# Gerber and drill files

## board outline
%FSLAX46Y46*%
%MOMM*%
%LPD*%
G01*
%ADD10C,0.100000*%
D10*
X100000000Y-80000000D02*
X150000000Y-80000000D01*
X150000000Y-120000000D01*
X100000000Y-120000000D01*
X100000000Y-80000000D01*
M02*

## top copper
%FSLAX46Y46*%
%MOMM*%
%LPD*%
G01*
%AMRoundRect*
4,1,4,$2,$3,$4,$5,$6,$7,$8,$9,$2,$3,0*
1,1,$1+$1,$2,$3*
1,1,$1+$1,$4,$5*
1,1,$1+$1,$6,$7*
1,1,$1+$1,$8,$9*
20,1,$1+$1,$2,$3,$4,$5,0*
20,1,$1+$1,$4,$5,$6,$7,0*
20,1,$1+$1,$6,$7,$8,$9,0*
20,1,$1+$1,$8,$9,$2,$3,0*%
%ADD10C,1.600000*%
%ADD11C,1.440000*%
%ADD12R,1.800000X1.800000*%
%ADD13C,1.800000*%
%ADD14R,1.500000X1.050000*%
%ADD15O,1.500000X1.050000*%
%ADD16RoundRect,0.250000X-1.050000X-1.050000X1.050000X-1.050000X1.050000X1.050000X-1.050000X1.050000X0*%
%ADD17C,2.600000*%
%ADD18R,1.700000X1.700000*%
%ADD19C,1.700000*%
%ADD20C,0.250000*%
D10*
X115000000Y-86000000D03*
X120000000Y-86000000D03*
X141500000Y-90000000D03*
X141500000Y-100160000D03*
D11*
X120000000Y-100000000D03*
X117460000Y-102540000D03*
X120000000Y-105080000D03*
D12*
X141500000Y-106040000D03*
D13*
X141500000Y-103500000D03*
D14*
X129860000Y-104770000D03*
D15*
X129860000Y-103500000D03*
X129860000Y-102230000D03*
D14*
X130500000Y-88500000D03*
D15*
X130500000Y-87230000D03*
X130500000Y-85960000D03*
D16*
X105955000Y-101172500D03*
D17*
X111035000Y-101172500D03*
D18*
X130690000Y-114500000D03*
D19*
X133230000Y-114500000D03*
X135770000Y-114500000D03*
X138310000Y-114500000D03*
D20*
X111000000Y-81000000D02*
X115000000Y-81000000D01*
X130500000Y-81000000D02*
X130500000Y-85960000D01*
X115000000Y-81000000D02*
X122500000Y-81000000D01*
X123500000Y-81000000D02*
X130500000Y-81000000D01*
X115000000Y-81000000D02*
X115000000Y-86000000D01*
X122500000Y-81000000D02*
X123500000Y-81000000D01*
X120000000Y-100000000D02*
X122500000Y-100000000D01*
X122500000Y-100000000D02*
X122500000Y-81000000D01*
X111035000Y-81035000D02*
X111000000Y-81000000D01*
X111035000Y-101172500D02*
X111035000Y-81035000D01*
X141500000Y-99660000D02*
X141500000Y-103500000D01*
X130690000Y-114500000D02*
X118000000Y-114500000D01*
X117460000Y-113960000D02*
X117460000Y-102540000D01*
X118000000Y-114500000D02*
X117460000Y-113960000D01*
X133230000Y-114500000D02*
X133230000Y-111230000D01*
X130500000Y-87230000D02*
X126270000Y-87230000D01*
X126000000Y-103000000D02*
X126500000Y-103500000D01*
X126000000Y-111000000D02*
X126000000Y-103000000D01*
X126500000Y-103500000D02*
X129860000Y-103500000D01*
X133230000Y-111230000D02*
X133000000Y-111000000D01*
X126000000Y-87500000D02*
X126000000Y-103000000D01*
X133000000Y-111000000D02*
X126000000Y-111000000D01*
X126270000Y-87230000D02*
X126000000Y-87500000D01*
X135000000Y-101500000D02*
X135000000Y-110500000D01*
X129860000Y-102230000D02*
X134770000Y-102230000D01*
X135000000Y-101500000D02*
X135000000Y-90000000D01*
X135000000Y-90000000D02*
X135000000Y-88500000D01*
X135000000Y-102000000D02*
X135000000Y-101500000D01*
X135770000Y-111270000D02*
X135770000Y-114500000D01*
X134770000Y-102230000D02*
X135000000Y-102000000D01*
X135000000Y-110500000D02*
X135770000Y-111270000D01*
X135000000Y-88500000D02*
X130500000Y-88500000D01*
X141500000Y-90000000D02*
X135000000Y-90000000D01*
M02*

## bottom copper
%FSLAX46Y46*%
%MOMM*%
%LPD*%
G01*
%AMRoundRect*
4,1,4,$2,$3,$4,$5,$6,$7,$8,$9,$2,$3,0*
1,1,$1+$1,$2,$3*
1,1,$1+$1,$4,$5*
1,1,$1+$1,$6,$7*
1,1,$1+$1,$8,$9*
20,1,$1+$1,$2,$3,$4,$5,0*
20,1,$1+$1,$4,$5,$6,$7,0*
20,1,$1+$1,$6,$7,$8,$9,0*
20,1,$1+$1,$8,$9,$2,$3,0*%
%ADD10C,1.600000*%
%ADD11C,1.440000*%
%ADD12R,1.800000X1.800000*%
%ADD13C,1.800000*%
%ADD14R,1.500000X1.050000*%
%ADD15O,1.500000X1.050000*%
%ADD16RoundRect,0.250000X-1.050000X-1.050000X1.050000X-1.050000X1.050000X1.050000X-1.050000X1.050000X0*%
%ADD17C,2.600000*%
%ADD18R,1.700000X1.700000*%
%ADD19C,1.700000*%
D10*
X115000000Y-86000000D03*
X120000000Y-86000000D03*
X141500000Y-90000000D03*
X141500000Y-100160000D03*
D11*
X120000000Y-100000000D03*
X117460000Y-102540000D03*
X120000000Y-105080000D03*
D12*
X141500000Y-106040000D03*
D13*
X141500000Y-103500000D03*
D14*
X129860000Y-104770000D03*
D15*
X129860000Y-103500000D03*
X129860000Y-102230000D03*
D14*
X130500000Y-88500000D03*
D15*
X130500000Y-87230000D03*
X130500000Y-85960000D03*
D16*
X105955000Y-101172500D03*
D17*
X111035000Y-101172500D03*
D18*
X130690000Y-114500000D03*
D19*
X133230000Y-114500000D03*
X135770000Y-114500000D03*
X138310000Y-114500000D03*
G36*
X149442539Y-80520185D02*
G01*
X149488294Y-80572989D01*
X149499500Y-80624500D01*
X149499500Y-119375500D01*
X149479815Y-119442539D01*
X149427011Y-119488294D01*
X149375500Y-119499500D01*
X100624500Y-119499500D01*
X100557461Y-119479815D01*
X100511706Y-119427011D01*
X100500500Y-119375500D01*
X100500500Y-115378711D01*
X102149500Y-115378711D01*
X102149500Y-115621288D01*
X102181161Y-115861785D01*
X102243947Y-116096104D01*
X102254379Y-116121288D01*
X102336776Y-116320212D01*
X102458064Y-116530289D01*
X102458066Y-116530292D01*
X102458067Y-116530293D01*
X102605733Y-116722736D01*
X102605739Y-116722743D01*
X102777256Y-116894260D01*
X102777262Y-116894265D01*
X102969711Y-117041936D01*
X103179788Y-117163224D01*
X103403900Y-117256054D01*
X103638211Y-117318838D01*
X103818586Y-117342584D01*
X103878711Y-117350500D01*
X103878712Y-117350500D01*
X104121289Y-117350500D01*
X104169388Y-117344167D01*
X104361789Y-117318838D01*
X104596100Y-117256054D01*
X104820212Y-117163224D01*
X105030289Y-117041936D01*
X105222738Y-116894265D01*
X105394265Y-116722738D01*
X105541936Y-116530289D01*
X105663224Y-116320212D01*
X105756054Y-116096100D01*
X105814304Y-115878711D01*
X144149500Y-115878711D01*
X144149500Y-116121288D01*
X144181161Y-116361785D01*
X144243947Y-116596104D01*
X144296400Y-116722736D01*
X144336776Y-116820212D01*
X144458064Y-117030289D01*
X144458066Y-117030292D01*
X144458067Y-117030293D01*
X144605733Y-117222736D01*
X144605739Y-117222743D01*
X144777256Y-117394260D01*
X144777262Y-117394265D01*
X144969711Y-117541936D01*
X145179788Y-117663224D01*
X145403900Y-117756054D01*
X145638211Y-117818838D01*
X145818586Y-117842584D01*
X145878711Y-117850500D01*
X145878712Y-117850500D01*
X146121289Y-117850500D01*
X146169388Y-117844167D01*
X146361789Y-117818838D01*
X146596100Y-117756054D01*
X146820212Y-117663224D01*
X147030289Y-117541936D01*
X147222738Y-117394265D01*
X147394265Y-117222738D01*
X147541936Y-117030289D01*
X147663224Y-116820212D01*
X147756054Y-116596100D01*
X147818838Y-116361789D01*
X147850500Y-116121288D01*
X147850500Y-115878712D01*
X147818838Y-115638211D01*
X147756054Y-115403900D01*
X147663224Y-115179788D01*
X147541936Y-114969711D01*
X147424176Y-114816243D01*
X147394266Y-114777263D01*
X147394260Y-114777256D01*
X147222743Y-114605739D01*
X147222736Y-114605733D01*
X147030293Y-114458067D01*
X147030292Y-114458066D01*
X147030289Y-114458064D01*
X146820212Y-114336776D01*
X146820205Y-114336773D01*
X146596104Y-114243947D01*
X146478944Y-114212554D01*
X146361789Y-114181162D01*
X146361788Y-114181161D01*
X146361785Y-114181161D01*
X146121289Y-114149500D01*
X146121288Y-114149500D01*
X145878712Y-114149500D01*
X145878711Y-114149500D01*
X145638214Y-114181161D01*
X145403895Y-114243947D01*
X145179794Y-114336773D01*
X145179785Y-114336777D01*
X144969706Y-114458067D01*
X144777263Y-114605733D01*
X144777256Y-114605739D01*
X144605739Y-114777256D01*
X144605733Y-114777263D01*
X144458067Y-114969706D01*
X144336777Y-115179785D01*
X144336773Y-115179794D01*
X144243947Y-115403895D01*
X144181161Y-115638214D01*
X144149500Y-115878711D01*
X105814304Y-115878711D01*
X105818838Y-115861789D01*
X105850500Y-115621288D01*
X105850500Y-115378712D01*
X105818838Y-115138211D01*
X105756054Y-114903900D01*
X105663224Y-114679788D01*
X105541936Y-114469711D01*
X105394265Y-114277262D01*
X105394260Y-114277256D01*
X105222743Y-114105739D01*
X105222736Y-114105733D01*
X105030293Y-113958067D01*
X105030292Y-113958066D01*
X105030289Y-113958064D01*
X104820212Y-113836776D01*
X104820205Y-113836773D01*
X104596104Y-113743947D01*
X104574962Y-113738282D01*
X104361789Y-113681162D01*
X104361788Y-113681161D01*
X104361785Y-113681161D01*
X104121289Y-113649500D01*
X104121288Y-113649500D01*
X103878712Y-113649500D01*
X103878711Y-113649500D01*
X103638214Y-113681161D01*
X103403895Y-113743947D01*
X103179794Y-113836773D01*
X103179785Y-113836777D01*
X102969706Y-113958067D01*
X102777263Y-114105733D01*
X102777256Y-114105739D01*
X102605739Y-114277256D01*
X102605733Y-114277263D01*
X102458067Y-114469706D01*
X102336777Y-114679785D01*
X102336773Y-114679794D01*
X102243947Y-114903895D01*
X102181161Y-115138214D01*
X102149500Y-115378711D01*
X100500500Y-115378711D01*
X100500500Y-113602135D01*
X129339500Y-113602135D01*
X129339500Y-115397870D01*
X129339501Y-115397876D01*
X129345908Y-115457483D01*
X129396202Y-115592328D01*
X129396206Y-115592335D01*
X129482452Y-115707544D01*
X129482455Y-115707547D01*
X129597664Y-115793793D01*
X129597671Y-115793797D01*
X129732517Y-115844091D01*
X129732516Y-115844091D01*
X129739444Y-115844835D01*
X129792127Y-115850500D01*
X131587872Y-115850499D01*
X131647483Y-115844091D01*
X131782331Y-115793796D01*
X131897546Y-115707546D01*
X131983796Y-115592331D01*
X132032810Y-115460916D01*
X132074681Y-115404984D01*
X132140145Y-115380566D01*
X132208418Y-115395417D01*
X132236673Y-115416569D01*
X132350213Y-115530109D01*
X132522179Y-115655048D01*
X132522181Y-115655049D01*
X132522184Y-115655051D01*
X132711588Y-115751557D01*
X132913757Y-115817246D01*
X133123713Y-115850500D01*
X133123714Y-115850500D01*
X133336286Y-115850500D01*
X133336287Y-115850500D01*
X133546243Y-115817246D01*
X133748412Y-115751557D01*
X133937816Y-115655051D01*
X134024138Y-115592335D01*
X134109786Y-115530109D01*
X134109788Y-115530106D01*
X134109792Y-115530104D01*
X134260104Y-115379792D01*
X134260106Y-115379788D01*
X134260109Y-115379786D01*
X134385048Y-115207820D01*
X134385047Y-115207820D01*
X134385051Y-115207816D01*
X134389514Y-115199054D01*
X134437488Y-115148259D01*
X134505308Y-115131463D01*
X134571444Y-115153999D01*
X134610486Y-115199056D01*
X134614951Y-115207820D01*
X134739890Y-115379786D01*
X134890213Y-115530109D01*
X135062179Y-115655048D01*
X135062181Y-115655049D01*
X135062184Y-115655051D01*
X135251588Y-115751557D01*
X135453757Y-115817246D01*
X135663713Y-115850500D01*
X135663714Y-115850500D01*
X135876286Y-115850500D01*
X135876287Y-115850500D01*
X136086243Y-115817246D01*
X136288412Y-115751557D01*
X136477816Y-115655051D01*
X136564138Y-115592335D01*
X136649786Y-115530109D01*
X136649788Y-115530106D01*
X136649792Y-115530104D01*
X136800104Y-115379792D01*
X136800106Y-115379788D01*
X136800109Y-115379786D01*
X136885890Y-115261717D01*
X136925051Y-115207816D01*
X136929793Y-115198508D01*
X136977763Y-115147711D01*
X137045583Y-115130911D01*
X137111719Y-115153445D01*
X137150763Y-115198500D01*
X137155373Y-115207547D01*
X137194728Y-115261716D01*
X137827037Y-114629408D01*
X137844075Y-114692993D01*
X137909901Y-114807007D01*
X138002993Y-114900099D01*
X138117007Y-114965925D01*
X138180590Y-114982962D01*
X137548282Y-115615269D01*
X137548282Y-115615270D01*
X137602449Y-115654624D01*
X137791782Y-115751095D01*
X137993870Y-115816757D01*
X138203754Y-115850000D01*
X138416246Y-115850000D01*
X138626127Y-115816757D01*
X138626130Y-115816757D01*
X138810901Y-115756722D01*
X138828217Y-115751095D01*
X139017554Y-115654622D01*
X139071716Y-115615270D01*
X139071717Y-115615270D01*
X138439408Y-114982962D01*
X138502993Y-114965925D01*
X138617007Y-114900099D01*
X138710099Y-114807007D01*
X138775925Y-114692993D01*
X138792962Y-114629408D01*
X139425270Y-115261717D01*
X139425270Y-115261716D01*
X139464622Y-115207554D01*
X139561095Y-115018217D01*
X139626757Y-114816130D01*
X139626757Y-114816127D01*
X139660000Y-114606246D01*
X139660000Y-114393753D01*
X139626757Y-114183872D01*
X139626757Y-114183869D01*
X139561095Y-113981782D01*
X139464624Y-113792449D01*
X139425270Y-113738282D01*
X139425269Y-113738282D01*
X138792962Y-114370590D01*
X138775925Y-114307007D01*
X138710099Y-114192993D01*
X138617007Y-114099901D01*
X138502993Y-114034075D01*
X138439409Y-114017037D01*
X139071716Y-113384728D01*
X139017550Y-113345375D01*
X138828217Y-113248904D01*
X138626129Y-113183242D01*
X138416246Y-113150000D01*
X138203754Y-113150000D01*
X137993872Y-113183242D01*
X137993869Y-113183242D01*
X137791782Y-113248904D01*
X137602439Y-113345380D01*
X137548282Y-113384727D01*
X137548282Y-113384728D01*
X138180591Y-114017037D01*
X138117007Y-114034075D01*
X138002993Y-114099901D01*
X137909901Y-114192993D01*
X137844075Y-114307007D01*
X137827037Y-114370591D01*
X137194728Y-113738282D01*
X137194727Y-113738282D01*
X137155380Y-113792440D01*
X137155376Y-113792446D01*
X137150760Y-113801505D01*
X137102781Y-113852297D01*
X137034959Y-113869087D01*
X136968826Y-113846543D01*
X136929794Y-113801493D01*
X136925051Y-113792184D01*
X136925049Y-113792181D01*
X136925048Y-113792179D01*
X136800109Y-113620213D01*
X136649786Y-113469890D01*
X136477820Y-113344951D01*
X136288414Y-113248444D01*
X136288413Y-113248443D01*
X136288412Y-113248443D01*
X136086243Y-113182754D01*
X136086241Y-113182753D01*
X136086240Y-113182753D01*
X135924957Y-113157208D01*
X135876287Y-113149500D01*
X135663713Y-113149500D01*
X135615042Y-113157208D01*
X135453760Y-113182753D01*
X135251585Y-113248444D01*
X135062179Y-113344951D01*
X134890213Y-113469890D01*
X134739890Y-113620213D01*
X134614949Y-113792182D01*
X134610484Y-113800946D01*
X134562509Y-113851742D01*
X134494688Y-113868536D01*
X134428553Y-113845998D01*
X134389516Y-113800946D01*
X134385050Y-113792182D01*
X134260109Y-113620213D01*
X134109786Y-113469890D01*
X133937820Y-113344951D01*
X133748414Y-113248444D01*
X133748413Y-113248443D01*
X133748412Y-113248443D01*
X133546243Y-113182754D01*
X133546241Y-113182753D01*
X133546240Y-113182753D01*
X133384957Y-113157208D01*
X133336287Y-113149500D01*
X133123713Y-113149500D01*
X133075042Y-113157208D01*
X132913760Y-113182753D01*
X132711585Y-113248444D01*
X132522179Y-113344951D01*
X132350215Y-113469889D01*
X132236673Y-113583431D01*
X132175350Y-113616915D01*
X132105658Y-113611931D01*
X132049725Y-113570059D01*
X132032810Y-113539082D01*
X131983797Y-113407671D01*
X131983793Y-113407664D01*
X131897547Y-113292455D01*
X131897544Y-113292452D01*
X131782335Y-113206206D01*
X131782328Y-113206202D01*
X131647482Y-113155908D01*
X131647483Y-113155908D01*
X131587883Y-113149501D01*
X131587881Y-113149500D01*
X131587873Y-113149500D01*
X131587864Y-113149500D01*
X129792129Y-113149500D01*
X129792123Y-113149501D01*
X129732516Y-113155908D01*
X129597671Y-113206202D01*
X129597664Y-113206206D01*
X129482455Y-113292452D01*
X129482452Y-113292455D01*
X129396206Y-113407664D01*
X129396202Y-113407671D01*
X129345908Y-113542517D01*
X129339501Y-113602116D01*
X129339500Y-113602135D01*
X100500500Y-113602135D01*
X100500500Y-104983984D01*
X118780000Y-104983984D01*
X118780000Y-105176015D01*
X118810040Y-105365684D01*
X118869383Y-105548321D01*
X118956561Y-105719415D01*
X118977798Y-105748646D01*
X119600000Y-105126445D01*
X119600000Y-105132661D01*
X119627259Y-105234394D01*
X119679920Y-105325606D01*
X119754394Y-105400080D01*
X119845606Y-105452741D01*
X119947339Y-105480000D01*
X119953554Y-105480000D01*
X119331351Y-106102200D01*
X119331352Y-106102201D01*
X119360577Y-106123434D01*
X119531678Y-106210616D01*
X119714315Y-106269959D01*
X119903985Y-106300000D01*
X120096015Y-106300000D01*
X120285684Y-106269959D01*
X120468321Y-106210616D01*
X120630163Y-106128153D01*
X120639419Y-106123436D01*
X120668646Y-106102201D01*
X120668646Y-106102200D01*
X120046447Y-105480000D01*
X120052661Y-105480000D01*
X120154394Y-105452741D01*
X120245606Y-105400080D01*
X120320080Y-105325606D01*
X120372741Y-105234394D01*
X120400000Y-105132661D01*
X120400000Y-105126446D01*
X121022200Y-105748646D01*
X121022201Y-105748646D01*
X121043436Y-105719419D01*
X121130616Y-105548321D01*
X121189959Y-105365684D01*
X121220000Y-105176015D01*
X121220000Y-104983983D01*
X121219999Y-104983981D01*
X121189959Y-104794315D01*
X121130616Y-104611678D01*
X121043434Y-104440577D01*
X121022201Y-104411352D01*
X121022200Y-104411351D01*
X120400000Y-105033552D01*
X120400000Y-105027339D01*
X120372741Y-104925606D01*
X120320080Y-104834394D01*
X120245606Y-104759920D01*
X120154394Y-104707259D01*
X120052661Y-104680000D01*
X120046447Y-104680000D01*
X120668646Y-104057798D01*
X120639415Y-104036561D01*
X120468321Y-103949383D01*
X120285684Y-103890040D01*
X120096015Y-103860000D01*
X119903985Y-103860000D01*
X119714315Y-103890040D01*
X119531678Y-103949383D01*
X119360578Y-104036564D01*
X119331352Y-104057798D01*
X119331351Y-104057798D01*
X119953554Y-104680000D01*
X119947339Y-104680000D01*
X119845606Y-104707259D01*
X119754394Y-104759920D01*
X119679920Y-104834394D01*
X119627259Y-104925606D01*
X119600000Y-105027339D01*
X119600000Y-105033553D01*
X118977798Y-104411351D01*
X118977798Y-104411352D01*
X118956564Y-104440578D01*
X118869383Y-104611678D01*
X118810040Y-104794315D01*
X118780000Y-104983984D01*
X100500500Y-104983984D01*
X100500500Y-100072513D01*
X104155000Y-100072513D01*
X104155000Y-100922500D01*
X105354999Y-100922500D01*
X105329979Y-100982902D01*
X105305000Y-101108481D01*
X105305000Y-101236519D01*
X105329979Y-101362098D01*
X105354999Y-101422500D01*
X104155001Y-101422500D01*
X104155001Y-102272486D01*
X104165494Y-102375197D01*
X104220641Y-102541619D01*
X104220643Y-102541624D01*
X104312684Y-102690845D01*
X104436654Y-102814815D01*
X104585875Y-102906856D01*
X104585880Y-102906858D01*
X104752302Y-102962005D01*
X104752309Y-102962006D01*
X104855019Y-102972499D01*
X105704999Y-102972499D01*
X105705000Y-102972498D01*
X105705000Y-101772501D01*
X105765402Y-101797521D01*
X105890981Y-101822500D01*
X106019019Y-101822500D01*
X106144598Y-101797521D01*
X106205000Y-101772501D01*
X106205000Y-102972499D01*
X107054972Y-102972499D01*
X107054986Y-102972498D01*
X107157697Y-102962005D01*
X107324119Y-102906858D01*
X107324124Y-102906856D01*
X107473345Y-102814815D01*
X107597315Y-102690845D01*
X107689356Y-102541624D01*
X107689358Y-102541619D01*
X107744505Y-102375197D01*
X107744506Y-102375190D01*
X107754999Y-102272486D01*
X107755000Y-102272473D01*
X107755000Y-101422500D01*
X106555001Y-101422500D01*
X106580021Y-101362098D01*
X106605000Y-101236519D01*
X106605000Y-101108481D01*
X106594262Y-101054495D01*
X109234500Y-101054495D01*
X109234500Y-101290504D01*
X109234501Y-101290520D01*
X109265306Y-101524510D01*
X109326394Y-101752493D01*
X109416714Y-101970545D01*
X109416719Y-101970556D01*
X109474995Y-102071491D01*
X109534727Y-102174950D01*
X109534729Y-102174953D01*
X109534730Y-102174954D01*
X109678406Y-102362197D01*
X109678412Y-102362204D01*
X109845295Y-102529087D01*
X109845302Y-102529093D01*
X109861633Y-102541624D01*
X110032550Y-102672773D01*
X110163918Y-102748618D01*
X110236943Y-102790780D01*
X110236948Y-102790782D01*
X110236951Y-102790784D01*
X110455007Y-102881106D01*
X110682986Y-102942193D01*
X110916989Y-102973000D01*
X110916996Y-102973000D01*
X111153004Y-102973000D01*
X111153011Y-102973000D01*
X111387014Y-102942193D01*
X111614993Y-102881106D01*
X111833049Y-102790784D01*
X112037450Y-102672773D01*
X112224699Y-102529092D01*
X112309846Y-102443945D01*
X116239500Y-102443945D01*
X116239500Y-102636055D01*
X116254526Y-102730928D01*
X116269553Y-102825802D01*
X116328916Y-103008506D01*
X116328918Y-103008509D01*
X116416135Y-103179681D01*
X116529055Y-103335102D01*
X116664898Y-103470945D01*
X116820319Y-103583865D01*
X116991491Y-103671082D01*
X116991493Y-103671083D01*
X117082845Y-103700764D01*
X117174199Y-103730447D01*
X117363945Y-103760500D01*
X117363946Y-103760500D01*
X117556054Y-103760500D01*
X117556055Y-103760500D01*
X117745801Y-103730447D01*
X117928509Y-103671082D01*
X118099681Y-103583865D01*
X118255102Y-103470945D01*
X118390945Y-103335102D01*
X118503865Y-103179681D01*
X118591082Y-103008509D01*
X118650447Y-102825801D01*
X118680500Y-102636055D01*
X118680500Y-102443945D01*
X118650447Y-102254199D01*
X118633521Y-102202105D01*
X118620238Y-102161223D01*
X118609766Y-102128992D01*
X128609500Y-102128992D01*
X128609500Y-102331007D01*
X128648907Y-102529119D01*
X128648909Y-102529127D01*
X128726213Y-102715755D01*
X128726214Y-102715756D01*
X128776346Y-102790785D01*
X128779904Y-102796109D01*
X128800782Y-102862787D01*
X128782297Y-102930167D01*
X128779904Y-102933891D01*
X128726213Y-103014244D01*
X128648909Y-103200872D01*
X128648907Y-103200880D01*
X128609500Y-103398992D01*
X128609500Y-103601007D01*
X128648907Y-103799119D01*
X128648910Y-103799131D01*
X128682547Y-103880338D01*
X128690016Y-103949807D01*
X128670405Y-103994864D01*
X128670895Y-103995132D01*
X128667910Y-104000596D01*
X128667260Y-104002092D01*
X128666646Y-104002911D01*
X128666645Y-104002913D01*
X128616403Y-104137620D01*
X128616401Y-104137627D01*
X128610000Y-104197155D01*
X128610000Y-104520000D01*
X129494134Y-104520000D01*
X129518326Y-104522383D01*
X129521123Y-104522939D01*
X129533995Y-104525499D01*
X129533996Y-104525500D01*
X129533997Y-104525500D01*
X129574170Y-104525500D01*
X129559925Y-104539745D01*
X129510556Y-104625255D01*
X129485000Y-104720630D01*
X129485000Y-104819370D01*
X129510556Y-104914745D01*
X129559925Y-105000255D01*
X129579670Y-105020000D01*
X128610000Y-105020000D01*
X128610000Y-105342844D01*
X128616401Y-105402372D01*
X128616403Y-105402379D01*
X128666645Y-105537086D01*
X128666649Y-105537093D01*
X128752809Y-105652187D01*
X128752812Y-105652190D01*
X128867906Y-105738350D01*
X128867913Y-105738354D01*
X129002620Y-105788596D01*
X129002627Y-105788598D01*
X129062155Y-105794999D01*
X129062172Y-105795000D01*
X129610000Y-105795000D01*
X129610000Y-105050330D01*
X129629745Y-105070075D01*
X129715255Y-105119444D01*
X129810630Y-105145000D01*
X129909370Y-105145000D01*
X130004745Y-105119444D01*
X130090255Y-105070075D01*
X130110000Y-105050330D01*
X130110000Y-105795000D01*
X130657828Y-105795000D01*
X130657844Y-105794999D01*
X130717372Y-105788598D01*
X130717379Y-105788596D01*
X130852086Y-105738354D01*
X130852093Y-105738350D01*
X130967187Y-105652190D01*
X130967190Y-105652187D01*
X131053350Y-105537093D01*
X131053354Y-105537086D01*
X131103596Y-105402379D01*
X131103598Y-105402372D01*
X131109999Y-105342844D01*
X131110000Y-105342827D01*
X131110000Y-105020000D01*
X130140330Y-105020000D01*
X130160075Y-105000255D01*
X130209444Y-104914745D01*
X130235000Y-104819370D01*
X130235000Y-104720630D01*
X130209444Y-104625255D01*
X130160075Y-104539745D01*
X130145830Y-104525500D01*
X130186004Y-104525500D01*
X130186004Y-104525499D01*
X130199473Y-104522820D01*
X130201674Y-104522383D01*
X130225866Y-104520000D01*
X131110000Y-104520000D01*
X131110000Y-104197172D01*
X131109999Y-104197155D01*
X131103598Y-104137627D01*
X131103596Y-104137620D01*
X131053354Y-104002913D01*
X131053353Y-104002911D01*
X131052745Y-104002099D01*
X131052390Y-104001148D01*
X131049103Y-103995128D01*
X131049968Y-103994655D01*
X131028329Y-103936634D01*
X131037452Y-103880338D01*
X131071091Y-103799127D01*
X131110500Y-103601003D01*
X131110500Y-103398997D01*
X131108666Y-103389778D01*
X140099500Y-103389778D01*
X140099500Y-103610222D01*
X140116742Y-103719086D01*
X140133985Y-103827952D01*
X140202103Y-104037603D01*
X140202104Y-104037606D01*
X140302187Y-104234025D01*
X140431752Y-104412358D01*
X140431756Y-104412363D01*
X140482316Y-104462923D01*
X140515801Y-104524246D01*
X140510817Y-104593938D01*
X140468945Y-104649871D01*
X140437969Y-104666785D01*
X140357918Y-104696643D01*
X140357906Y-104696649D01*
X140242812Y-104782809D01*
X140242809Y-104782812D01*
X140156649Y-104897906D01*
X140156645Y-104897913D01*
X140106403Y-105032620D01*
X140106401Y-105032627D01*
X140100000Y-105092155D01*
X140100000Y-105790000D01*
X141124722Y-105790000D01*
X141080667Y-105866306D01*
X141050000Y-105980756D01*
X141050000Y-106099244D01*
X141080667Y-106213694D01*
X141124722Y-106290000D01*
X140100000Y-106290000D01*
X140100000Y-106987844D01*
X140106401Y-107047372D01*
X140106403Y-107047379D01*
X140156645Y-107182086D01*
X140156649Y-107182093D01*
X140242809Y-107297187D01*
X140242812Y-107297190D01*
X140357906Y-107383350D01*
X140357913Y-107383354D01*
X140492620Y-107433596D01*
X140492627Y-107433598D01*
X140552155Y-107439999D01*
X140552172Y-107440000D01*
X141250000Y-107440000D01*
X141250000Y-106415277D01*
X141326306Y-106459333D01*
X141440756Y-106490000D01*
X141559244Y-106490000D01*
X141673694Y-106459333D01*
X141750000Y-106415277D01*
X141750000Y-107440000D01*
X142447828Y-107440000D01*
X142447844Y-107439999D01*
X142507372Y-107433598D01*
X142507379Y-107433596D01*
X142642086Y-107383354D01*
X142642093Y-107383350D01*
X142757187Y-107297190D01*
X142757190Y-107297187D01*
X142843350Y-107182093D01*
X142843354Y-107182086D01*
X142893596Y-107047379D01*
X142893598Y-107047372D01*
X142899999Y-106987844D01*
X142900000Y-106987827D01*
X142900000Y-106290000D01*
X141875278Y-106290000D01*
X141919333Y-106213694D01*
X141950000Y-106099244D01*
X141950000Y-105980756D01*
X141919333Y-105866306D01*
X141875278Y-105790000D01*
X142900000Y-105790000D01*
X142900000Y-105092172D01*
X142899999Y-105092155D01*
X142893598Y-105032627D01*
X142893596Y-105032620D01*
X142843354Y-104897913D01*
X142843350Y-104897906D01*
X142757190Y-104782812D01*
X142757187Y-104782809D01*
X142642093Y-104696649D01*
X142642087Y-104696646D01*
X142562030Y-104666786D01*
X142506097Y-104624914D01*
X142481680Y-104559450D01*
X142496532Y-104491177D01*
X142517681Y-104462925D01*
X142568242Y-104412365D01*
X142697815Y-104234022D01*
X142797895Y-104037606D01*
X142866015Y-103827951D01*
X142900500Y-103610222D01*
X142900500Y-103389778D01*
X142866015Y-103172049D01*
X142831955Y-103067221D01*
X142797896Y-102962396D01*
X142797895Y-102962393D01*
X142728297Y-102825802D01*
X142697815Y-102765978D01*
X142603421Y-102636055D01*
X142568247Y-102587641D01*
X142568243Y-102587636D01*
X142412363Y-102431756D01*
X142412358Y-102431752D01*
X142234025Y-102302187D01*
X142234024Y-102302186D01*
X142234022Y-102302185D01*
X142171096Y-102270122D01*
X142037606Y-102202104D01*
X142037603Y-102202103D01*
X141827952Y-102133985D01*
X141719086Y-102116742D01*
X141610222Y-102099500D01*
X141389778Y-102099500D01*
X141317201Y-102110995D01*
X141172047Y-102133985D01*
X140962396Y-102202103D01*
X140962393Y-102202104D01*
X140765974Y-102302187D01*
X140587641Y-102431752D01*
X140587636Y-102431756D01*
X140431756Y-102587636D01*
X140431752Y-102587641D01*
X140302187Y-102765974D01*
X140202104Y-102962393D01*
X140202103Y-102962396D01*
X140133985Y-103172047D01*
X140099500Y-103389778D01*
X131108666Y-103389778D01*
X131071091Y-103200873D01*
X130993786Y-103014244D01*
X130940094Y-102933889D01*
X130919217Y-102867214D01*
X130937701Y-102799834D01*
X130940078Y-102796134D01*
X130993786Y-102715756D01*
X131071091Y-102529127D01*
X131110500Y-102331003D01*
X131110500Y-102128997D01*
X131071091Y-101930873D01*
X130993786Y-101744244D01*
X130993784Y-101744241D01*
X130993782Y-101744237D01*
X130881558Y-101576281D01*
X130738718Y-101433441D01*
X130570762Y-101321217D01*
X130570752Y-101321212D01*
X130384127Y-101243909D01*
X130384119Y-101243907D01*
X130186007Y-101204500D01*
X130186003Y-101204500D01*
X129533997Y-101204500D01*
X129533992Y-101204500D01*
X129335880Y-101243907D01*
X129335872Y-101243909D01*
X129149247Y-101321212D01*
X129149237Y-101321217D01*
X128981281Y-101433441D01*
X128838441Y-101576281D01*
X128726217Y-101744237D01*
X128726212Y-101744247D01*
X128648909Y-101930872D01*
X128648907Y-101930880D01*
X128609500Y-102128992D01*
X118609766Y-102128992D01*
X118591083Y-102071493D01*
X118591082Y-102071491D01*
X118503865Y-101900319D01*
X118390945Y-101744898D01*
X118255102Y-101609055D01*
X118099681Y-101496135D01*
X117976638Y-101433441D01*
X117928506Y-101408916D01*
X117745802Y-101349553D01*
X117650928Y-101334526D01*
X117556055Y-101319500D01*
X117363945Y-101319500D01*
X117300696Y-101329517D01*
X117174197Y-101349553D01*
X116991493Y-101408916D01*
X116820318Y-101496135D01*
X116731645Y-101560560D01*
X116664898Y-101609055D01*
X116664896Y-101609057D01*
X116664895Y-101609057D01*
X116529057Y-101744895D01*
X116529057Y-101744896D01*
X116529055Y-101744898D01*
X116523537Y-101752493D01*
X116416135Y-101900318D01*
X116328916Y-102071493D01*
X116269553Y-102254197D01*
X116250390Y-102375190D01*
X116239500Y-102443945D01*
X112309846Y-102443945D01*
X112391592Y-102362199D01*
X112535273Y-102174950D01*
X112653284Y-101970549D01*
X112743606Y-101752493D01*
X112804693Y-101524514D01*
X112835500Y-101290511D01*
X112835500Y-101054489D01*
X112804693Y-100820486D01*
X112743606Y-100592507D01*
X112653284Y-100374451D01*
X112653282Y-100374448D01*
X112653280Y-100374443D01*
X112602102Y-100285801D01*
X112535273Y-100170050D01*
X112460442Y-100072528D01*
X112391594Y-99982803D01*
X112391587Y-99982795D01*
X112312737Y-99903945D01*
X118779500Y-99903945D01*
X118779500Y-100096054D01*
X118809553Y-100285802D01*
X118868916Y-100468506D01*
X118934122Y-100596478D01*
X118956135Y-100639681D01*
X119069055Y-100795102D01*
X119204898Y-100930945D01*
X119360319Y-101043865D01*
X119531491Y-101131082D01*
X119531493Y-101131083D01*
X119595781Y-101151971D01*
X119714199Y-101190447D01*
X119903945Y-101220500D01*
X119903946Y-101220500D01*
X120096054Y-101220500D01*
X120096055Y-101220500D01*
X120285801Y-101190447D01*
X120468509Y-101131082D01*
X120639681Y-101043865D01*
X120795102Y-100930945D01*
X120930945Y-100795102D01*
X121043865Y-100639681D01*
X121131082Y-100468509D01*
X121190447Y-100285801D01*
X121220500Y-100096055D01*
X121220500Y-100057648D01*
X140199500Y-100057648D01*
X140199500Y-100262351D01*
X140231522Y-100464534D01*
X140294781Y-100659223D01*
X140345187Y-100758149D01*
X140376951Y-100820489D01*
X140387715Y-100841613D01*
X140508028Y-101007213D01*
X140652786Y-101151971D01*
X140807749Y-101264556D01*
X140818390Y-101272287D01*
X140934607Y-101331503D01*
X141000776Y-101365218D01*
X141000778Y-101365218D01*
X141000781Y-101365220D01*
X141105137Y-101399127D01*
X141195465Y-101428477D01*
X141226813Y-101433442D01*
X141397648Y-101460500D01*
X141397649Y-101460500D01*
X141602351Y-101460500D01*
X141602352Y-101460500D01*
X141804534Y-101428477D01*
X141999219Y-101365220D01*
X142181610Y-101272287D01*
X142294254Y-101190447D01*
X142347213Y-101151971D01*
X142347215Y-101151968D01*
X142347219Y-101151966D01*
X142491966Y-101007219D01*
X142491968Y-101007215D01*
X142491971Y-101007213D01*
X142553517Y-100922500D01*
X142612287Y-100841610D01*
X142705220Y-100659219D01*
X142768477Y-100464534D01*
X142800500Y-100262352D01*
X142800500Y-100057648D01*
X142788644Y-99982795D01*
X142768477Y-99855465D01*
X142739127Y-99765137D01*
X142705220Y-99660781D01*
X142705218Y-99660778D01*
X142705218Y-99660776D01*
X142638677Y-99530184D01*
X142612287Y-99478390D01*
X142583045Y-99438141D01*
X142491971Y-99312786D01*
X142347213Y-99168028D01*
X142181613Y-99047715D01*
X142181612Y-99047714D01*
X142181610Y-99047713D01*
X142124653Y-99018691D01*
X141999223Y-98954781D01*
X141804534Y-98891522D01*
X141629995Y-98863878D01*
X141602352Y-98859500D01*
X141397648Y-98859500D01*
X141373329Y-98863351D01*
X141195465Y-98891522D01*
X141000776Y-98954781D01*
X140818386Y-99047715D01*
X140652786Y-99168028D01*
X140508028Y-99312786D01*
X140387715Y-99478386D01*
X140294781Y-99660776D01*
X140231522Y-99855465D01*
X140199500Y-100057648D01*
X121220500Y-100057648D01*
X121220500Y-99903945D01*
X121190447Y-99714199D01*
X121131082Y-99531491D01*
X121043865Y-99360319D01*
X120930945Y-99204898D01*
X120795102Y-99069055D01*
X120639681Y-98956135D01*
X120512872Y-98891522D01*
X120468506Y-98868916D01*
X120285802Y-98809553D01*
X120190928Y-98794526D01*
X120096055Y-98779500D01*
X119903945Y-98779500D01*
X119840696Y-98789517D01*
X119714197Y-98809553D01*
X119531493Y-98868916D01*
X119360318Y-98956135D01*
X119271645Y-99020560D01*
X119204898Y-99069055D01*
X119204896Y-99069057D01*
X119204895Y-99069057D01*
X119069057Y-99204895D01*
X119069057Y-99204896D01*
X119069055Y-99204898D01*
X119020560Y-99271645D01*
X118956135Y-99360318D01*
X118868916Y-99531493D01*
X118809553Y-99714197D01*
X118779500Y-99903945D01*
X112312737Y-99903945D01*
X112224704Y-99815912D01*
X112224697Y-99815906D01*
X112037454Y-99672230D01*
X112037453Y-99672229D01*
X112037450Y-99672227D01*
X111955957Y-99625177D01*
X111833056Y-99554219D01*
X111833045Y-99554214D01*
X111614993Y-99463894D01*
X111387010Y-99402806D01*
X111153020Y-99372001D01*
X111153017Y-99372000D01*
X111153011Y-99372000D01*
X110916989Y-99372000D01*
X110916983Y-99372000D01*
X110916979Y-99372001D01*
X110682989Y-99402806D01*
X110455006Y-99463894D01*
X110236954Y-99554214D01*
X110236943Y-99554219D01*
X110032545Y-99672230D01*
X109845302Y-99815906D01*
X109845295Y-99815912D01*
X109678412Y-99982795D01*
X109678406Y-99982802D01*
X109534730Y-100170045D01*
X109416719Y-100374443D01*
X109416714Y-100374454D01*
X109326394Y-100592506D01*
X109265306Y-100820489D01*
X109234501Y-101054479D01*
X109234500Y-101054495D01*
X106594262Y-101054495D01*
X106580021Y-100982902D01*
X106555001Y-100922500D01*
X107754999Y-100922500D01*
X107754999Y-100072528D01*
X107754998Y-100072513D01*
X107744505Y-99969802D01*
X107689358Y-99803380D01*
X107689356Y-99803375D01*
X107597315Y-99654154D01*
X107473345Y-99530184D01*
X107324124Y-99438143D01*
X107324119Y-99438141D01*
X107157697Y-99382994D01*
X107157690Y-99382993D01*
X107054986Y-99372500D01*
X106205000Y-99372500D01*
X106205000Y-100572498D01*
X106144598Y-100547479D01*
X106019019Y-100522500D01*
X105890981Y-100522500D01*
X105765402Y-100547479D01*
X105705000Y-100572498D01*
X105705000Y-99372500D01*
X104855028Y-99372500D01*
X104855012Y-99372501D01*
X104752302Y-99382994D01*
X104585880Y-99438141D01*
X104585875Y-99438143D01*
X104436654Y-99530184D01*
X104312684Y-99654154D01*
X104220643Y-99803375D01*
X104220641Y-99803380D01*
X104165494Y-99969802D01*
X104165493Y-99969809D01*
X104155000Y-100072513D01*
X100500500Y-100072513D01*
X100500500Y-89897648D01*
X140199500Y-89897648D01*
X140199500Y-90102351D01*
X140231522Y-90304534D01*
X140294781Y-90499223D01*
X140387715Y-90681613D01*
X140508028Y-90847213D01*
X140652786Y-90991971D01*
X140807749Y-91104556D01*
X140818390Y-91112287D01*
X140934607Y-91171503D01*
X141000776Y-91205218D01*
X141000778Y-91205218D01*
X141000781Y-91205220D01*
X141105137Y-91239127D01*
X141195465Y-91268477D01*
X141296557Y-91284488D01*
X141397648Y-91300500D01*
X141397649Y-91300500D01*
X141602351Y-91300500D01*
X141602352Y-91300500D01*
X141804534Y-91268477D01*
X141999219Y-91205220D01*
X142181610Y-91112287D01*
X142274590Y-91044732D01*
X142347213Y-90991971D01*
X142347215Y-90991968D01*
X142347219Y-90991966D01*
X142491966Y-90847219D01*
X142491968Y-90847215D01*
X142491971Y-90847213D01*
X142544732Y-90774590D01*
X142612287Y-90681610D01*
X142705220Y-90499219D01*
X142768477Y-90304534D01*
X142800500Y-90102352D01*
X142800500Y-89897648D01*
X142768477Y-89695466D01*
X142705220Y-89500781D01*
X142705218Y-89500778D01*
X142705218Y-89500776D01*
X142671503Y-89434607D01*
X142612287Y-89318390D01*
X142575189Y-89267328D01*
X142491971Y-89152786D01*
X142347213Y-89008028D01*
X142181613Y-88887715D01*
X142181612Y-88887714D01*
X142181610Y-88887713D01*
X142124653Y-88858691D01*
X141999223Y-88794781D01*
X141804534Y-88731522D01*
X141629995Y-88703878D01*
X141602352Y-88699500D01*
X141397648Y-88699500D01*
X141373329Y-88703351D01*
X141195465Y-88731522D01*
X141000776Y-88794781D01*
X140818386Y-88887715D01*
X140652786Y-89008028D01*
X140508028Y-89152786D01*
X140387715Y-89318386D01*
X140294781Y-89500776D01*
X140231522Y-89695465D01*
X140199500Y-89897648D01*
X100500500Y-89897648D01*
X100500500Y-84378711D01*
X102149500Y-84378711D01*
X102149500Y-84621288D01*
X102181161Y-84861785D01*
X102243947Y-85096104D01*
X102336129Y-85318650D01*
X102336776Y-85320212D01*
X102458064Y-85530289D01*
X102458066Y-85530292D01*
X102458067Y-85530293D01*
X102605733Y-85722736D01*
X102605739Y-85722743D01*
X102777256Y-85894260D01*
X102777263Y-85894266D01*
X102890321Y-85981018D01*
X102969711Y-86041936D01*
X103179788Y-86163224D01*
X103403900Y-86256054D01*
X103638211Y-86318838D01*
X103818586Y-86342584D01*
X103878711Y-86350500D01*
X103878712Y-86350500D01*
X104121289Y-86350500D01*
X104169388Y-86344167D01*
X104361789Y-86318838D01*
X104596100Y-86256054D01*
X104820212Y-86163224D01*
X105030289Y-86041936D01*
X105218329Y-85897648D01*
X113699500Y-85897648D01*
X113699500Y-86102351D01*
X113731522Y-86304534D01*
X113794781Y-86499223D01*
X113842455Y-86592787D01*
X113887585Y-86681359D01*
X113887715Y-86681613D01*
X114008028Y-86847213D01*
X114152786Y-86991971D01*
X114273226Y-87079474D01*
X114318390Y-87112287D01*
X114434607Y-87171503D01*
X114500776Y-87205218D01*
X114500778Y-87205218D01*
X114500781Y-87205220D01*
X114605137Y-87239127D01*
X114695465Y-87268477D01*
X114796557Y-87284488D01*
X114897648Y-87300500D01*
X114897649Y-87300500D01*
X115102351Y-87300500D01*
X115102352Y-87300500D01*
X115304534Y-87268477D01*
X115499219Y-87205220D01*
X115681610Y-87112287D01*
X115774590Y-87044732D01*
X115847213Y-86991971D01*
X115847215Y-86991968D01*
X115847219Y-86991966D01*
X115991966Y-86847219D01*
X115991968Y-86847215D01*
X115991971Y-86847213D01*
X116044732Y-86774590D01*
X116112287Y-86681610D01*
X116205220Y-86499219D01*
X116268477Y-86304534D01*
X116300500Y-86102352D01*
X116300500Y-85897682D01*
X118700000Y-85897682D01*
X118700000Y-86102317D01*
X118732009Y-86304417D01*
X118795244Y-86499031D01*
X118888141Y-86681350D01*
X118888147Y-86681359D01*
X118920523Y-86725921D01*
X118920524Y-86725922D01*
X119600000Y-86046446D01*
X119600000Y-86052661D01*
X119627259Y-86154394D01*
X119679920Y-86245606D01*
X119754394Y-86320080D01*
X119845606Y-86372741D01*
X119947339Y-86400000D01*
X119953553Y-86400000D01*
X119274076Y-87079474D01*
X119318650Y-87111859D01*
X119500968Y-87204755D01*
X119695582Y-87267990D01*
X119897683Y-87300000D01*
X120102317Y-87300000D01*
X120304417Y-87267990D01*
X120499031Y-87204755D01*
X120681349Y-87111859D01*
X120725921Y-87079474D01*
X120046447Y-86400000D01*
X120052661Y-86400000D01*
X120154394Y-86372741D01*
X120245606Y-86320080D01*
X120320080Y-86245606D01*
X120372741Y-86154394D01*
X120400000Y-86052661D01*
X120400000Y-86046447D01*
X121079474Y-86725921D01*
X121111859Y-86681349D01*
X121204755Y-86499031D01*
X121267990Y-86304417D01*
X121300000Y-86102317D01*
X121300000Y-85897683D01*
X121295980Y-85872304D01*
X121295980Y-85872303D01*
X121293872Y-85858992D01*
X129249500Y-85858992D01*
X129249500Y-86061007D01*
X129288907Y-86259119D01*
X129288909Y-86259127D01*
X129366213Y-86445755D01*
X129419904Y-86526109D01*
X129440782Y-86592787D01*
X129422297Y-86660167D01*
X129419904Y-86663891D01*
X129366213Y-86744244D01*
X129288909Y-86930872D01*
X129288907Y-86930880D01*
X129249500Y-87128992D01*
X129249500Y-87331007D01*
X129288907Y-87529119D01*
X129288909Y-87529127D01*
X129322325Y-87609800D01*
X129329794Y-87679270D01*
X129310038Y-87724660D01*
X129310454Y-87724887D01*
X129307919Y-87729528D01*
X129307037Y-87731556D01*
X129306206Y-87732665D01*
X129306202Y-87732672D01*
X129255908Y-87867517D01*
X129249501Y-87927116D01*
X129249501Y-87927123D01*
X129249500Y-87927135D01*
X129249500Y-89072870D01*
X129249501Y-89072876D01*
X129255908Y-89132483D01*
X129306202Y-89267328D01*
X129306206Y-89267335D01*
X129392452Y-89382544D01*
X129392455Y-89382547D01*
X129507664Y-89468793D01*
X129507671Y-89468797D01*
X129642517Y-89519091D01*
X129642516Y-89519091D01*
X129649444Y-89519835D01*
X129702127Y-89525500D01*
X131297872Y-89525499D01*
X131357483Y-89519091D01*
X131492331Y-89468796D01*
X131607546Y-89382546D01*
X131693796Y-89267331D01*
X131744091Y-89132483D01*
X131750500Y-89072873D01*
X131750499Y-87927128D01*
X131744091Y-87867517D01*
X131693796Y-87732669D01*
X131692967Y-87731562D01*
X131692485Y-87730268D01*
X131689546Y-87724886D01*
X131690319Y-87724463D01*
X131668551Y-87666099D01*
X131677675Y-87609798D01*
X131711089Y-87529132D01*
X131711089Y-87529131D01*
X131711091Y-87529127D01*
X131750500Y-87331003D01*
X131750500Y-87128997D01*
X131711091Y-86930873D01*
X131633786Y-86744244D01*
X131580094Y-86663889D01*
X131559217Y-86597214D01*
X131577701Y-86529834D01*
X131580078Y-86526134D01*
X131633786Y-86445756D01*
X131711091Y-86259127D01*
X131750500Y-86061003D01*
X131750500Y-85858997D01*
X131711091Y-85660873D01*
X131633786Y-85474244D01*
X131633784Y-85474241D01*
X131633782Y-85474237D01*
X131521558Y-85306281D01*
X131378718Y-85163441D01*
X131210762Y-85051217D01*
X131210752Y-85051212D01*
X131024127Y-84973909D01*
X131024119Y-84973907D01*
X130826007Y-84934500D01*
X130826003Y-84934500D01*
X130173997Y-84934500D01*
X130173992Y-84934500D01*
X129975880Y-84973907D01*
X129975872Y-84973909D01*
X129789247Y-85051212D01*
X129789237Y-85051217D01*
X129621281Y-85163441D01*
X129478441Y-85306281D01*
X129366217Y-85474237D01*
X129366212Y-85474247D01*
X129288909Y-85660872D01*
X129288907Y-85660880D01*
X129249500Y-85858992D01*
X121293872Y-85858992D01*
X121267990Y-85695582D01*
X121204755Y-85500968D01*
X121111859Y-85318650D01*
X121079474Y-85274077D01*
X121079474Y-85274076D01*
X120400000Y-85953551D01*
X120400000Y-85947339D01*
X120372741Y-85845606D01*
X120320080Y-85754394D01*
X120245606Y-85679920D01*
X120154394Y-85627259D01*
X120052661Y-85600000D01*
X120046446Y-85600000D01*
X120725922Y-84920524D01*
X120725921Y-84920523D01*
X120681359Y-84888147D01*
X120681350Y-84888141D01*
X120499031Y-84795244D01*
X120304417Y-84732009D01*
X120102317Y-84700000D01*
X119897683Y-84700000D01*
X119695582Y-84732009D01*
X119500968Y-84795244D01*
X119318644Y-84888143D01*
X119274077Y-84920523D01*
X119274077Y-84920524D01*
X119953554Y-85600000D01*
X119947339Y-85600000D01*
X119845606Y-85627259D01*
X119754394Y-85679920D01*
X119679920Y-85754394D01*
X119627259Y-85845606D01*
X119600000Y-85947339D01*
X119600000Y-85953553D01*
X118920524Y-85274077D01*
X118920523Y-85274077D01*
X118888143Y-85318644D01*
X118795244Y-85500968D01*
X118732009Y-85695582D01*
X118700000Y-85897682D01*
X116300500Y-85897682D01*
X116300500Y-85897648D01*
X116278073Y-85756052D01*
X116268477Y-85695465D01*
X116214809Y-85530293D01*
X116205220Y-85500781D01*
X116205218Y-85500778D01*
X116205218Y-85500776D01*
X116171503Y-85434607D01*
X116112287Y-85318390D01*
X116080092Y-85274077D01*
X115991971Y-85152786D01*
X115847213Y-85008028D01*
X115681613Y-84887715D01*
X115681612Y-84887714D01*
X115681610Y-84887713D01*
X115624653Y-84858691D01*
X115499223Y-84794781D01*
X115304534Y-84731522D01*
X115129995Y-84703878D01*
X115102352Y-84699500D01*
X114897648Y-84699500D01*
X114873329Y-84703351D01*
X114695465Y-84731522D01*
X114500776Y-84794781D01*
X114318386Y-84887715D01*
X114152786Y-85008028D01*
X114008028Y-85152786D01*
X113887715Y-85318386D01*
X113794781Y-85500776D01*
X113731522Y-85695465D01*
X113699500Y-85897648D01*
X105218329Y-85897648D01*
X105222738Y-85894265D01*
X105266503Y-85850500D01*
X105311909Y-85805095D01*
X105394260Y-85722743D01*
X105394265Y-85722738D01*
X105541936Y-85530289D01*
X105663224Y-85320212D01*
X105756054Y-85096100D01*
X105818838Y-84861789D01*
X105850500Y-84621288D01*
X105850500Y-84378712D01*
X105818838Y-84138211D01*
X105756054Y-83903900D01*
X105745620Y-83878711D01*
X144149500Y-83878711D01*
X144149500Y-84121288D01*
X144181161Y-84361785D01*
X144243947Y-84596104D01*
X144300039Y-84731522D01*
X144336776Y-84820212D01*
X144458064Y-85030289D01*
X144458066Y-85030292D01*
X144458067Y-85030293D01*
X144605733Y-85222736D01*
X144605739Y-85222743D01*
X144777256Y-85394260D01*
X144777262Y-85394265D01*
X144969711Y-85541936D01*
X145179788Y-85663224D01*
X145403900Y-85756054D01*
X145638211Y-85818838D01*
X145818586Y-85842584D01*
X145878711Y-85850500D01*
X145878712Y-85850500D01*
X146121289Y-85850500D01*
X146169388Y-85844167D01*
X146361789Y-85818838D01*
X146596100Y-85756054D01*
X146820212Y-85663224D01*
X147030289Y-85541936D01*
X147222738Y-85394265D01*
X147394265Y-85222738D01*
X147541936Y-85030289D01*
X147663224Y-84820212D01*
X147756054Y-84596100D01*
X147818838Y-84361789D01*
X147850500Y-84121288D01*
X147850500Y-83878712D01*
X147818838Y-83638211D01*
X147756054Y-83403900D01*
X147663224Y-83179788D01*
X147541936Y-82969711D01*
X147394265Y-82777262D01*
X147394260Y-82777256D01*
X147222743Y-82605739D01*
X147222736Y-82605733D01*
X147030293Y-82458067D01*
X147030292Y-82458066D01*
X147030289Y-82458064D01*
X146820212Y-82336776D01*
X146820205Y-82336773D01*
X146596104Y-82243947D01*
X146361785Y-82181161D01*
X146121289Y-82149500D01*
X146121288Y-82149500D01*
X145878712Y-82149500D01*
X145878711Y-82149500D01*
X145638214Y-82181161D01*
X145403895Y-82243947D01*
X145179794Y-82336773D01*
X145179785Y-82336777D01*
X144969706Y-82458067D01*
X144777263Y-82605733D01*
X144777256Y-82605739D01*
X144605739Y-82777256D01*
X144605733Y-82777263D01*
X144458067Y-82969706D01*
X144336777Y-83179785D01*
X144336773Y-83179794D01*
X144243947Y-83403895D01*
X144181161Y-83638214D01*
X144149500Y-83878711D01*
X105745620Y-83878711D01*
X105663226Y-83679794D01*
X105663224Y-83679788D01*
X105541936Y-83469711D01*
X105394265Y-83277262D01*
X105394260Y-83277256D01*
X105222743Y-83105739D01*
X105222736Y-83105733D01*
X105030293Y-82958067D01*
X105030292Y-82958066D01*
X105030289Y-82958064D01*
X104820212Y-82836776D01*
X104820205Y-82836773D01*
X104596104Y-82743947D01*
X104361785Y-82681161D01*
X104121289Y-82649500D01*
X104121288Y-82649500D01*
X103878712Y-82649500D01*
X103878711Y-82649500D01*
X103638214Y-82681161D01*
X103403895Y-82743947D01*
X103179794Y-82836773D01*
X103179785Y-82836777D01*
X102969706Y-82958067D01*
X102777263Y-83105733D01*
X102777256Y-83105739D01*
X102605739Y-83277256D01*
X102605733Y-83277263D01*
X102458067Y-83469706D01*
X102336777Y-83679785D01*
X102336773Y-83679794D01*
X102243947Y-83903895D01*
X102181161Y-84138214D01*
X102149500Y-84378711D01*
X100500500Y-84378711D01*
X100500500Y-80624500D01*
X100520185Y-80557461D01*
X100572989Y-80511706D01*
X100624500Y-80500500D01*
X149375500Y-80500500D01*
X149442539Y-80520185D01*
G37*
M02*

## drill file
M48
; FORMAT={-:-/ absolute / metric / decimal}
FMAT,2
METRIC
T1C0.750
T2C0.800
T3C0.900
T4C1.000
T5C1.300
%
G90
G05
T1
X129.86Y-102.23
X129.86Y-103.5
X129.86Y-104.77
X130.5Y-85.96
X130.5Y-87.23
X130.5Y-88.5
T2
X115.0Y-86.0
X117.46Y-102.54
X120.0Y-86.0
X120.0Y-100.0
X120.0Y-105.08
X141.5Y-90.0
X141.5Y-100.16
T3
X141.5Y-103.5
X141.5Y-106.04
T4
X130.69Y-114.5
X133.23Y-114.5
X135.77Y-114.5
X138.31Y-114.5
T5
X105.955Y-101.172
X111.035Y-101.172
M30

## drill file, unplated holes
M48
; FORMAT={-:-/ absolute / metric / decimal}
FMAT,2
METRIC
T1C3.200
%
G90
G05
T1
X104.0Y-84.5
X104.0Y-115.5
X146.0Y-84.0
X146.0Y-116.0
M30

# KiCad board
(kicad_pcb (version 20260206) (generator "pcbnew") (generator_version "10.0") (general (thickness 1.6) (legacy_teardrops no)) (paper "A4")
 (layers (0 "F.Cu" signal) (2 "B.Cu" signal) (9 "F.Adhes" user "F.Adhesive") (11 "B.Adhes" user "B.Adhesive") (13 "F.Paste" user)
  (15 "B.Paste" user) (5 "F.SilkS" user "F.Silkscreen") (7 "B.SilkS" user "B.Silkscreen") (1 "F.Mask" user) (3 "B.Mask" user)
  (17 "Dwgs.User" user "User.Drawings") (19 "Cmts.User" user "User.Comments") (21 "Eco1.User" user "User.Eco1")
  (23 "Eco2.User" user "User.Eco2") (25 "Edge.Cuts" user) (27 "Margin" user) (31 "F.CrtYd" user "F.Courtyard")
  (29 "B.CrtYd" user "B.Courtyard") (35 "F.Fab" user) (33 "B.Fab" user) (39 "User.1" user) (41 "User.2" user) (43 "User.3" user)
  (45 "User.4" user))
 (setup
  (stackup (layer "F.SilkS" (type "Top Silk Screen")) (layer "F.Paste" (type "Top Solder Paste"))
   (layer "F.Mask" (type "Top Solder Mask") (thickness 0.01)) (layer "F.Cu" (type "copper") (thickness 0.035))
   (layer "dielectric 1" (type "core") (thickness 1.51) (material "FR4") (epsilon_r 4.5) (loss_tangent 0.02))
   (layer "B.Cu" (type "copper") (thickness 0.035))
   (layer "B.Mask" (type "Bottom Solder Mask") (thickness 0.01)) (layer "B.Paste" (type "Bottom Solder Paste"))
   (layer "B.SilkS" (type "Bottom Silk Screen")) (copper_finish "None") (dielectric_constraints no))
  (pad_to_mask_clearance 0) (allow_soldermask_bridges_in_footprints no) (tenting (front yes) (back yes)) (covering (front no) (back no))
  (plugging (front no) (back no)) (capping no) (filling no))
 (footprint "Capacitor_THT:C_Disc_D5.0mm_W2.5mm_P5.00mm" (layer "F.Cu") (at 115 86)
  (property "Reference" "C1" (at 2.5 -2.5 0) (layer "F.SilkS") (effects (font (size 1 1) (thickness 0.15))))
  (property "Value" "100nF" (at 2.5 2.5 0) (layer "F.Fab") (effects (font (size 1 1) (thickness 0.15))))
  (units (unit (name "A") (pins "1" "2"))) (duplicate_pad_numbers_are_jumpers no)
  (pad "1" thru_hole circle (at 0 0) (size 1.6 1.6) (drill 0.8) (layers "*.Cu" "*.Mask") (remove_unused_layers no) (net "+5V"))
  (pad "2" thru_hole circle (at 5 0) (size 1.6 1.6) (drill 0.8) (layers "*.Cu" "*.Mask") (remove_unused_layers no) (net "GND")))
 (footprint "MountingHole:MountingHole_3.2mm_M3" (layer "F.Cu") (at 104 115.5)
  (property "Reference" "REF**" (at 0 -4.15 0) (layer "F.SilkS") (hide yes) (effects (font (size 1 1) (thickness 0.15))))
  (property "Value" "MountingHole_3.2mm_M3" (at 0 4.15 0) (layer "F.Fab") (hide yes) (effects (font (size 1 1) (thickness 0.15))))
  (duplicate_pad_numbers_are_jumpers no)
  (pad "" np_thru_hole circle (at 0 0) (size 3.2 3.2) (drill 3.2) (layers "*.Cu" "*.Mask")))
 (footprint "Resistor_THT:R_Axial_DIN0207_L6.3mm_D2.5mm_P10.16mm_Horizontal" (layer "F.Cu") (at 141.5 90 -90)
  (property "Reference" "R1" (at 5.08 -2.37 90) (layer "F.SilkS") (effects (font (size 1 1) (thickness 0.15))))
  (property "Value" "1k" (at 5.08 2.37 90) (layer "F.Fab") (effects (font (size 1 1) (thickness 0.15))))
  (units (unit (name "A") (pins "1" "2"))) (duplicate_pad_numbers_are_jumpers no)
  (pad "1" thru_hole circle (at 0 0 270) (size 1.6 1.6) (drill 0.8) (layers "*.Cu" "*.Mask") (remove_unused_layers no) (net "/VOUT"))
  (pad "2" thru_hole circle (at 10.16 0 270) (size 1.6 1.6) (drill 0.8) (layers "*.Cu" "*.Mask") (remove_unused_layers no)
   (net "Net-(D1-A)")))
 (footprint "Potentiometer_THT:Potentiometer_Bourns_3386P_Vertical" (layer "F.Cu") (at 120 100 180)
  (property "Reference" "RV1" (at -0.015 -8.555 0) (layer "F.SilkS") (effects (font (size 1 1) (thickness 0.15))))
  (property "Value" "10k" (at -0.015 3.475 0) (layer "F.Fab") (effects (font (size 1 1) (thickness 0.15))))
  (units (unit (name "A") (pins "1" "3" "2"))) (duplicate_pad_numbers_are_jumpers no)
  (pad "1" thru_hole circle (at 0 0 180) (size 1.44 1.44) (drill 0.8) (layers "*.Cu" "*.Mask") (remove_unused_layers no) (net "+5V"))
  (pad "2" thru_hole circle (at 2.54 -2.54 180) (size 1.44 1.44) (drill 0.8) (layers "*.Cu" "*.Mask") (remove_unused_layers no)
   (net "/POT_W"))
  (pad "3" thru_hole circle (at 0 -5.08 180) (size 1.44 1.44) (drill 0.8) (layers "*.Cu" "*.Mask") (remove_unused_layers no) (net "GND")))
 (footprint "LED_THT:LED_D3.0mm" (layer "F.Cu") (at 141.5 106.04 90)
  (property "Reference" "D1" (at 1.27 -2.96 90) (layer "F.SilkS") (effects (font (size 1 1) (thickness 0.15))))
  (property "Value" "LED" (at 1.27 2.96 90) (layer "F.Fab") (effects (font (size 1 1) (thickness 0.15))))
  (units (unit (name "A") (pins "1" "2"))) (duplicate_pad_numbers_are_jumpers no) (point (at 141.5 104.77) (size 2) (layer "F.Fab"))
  (pad "1" thru_hole rect (at 0 0 90) (size 1.8 1.8) (drill 0.9) (layers "*.Cu" "*.Mask") (remove_unused_layers no) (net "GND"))
  (pad "2" thru_hole circle (at 2.54 0 90) (size 1.8 1.8) (drill 0.9) (layers "*.Cu" "*.Mask") (remove_unused_layers no) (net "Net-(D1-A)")))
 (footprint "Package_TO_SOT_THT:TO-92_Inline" (layer "F.Cu") (at 129.86 104.77 90)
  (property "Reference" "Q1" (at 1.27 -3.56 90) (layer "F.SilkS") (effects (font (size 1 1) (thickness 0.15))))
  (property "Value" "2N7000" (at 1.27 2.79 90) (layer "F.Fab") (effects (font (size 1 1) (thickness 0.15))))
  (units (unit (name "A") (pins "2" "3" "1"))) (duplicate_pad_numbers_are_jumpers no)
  (pad "1" thru_hole rect (at 0 0 90) (size 1.05 1.5) (drill 0.75) (layers "*.Cu" "*.Mask") (remove_unused_layers no) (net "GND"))
  (pad "2" thru_hole oval (at 1.27 0 90) (size 1.05 1.5) (drill 0.75) (layers "*.Cu" "*.Mask") (remove_unused_layers no) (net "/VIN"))
  (pad "3" thru_hole oval (at 2.54 0 90) (size 1.05 1.5) (drill 0.75) (layers "*.Cu" "*.Mask") (remove_unused_layers no) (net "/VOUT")))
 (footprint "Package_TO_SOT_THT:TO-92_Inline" (layer "F.Cu") (at 130.5 88.5 90)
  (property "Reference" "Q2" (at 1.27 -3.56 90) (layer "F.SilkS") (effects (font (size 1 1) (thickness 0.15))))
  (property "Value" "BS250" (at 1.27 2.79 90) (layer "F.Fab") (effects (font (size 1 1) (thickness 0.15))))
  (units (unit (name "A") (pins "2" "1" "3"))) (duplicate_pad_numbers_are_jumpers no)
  (pad "1" thru_hole rect (at 0 0 90) (size 1.05 1.5) (drill 0.75) (layers "*.Cu" "*.Mask") (remove_unused_layers no) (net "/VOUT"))
  (pad "2" thru_hole oval (at 1.27 0 90) (size 1.05 1.5) (drill 0.75) (layers "*.Cu" "*.Mask") (remove_unused_layers no) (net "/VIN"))
  (pad "3" thru_hole oval (at 2.54 0 90) (size 1.05 1.5) (drill 0.75) (layers "*.Cu" "*.Mask") (remove_unused_layers no) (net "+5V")))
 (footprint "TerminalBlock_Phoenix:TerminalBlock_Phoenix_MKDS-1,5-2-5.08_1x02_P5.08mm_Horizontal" (layer "F.Cu") (at 105.955 101.1725)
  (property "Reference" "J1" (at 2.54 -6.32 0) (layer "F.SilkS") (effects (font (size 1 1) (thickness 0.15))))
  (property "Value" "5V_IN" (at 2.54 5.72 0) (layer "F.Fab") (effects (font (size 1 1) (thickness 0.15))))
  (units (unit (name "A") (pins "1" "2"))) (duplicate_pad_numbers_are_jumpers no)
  (pad "1" thru_hole roundrect (at 0 0) (size 2.6 2.6) (drill 1.3) (layers "*.Cu" "*.Mask") (remove_unused_layers no)
   (roundrect_rratio 0.096154) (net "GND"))
  (pad "2" thru_hole circle (at 5.08 0) (size 2.6 2.6) (drill 1.3) (layers "*.Cu" "*.Mask") (remove_unused_layers no) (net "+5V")))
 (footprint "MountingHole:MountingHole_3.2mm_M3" (layer "F.Cu") (at 146 84)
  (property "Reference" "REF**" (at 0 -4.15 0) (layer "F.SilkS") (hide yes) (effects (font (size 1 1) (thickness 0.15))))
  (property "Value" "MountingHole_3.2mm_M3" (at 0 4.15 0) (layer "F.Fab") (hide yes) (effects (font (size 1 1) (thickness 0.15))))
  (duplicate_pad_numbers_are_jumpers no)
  (pad "" np_thru_hole circle (at 0 0) (size 3.2 3.2) (drill 3.2) (layers "*.Cu" "*.Mask")))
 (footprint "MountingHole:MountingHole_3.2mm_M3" (layer "F.Cu") (at 146 116)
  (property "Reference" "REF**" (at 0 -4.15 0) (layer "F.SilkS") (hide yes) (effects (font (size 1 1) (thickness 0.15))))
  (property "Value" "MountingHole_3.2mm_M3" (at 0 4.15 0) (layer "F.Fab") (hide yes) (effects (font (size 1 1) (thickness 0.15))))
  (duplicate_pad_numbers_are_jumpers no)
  (pad "" np_thru_hole circle (at 0 0) (size 3.2 3.2) (drill 3.2) (layers "*.Cu" "*.Mask")))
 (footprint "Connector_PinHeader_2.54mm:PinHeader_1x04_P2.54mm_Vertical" (layer "F.Cu") (at 130.69 114.5 90)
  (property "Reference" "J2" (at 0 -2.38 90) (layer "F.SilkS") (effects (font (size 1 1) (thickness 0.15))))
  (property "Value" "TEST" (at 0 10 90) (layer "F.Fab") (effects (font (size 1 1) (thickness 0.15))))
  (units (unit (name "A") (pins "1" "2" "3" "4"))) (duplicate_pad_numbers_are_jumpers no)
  (pad "1" thru_hole rect (at 0 0 90) (size 1.7 1.7) (drill 1) (layers "*.Cu" "*.Mask") (remove_unused_layers no) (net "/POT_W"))
  (pad "2" thru_hole circle (at 0 2.54 90) (size 1.7 1.7) (drill 1) (layers "*.Cu" "*.Mask") (remove_unused_layers no) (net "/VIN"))
  (pad "3" thru_hole circle (at 0 5.08 90) (size 1.7 1.7) (drill 1) (layers "*.Cu" "*.Mask") (remove_unused_layers no) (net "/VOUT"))
  (pad "4" thru_hole circle (at 0 7.62 90) (size 1.7 1.7) (drill 1) (layers "*.Cu" "*.Mask") (remove_unused_layers no) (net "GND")))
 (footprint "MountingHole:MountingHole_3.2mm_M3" (layer "F.Cu") (at 104 84.5)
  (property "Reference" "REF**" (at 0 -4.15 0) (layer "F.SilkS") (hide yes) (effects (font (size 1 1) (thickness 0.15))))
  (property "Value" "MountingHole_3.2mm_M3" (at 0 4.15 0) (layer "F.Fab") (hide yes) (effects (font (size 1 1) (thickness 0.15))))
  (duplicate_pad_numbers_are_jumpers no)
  (pad "" np_thru_hole circle (at 0 0) (size 3.2 3.2) (drill 3.2) (layers "*.Cu" "*.Mask")))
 (gr_rect (start 100 80) (end 150 120) (stroke (width 0.1) (type default)) (fill no) (layer "Edge.Cuts"))
 (segment (start 111 81) (end 115 81) (width 0.25) (layer "F.Cu") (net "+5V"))
 (segment (start 130.5 81) (end 130.5 85.96) (width 0.25) (layer "F.Cu") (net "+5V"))
 (segment (start 115 81) (end 122.5 81) (width 0.25) (layer "F.Cu") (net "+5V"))
 (segment (start 123.5 81) (end 130.5 81) (width 0.25) (layer "F.Cu") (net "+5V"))
 (segment (start 115 81) (end 115 86) (width 0.25) (layer "F.Cu") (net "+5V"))
 (segment (start 122.5 81) (end 123.5 81) (width 0.25) (layer "F.Cu") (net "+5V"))
 (segment (start 120 100) (end 122.5 100) (width 0.25) (layer "F.Cu") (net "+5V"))
 (segment (start 122.5 100) (end 122.5 81) (width 0.25) (layer "F.Cu") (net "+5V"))
 (segment (start 111.035 81.035) (end 111 81) (width 0.25) (layer "F.Cu") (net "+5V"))
 (segment (start 111.035 101.1725) (end 111.035 81.035) (width 0.25) (layer "F.Cu") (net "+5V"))
 (segment (start 135 101.5) (end 135 110.5) (width 0.25) (layer "F.Cu") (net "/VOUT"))
 (segment (start 129.86 102.23) (end 134.77 102.23) (width 0.25) (layer "F.Cu") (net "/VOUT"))
 (segment (start 135 101.5) (end 135 90) (width 0.25) (layer "F.Cu") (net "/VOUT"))
 (segment (start 135 90) (end 135 88.5) (width 0.25) (layer "F.Cu") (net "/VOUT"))
 (segment (start 135 102) (end 135 101.5) (width 0.25) (layer "F.Cu") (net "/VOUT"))
 (segment (start 135.77 111.27) (end 135.77 114.5) (width 0.25) (layer "F.Cu") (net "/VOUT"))
 (segment (start 134.77 102.23) (end 135 102) (width 0.25) (layer "F.Cu") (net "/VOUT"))
 (segment (start 135 110.5) (end 135.77 111.27) (width 0.25) (layer "F.Cu") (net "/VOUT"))
 (segment (start 135 88.5) (end 130.5 88.5) (width 0.25) (layer "F.Cu") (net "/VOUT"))
 (segment (start 141.5 90) (end 135 90) (width 0.25) (layer "F.Cu") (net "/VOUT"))
 (segment (start 141.5 99.66) (end 141.5 103.5) (width 0.25) (layer "F.Cu") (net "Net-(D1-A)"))
 (segment (start 130.69 114.5) (end 118 114.5) (width 0.25) (layer "F.Cu") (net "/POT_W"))
 (segment (start 117.46 113.96) (end 117.46 102.54) (width 0.25) (layer "F.Cu") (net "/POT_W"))
 (segment (start 118 114.5) (end 117.46 113.96) (width 0.25) (layer "F.Cu") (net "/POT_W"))
 (segment (start 133.23 114.5) (end 133.23 111.23) (width 0.25) (layer "F.Cu") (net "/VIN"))
 (segment (start 130.5 87.23) (end 126.27 87.23) (width 0.25) (layer "F.Cu") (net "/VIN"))
 (segment (start 126 103) (end 126.5 103.5) (width 0.25) (layer "F.Cu") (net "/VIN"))
 (segment (start 126 111) (end 126 103) (width 0.25) (layer "F.Cu") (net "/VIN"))
 (segment (start 126.5 103.5) (end 129.86 103.5) (width 0.25) (layer "F.Cu") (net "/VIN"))
 (segment (start 133.23 111.23) (end 133 111) (width 0.25) (layer "F.Cu") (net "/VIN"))
 (segment (start 126 87.5) (end 126 103) (width 0.25) (layer "F.Cu") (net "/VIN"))
 (segment (start 133 111) (end 126 111) (width 0.25) (layer "F.Cu") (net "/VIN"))
 (segment (start 126.27 87.23) (end 126 87.5) (width 0.25) (layer "F.Cu") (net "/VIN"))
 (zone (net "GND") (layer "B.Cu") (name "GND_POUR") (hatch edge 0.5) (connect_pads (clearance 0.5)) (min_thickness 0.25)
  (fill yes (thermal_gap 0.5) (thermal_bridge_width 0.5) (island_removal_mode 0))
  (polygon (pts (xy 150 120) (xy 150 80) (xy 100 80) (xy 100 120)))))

